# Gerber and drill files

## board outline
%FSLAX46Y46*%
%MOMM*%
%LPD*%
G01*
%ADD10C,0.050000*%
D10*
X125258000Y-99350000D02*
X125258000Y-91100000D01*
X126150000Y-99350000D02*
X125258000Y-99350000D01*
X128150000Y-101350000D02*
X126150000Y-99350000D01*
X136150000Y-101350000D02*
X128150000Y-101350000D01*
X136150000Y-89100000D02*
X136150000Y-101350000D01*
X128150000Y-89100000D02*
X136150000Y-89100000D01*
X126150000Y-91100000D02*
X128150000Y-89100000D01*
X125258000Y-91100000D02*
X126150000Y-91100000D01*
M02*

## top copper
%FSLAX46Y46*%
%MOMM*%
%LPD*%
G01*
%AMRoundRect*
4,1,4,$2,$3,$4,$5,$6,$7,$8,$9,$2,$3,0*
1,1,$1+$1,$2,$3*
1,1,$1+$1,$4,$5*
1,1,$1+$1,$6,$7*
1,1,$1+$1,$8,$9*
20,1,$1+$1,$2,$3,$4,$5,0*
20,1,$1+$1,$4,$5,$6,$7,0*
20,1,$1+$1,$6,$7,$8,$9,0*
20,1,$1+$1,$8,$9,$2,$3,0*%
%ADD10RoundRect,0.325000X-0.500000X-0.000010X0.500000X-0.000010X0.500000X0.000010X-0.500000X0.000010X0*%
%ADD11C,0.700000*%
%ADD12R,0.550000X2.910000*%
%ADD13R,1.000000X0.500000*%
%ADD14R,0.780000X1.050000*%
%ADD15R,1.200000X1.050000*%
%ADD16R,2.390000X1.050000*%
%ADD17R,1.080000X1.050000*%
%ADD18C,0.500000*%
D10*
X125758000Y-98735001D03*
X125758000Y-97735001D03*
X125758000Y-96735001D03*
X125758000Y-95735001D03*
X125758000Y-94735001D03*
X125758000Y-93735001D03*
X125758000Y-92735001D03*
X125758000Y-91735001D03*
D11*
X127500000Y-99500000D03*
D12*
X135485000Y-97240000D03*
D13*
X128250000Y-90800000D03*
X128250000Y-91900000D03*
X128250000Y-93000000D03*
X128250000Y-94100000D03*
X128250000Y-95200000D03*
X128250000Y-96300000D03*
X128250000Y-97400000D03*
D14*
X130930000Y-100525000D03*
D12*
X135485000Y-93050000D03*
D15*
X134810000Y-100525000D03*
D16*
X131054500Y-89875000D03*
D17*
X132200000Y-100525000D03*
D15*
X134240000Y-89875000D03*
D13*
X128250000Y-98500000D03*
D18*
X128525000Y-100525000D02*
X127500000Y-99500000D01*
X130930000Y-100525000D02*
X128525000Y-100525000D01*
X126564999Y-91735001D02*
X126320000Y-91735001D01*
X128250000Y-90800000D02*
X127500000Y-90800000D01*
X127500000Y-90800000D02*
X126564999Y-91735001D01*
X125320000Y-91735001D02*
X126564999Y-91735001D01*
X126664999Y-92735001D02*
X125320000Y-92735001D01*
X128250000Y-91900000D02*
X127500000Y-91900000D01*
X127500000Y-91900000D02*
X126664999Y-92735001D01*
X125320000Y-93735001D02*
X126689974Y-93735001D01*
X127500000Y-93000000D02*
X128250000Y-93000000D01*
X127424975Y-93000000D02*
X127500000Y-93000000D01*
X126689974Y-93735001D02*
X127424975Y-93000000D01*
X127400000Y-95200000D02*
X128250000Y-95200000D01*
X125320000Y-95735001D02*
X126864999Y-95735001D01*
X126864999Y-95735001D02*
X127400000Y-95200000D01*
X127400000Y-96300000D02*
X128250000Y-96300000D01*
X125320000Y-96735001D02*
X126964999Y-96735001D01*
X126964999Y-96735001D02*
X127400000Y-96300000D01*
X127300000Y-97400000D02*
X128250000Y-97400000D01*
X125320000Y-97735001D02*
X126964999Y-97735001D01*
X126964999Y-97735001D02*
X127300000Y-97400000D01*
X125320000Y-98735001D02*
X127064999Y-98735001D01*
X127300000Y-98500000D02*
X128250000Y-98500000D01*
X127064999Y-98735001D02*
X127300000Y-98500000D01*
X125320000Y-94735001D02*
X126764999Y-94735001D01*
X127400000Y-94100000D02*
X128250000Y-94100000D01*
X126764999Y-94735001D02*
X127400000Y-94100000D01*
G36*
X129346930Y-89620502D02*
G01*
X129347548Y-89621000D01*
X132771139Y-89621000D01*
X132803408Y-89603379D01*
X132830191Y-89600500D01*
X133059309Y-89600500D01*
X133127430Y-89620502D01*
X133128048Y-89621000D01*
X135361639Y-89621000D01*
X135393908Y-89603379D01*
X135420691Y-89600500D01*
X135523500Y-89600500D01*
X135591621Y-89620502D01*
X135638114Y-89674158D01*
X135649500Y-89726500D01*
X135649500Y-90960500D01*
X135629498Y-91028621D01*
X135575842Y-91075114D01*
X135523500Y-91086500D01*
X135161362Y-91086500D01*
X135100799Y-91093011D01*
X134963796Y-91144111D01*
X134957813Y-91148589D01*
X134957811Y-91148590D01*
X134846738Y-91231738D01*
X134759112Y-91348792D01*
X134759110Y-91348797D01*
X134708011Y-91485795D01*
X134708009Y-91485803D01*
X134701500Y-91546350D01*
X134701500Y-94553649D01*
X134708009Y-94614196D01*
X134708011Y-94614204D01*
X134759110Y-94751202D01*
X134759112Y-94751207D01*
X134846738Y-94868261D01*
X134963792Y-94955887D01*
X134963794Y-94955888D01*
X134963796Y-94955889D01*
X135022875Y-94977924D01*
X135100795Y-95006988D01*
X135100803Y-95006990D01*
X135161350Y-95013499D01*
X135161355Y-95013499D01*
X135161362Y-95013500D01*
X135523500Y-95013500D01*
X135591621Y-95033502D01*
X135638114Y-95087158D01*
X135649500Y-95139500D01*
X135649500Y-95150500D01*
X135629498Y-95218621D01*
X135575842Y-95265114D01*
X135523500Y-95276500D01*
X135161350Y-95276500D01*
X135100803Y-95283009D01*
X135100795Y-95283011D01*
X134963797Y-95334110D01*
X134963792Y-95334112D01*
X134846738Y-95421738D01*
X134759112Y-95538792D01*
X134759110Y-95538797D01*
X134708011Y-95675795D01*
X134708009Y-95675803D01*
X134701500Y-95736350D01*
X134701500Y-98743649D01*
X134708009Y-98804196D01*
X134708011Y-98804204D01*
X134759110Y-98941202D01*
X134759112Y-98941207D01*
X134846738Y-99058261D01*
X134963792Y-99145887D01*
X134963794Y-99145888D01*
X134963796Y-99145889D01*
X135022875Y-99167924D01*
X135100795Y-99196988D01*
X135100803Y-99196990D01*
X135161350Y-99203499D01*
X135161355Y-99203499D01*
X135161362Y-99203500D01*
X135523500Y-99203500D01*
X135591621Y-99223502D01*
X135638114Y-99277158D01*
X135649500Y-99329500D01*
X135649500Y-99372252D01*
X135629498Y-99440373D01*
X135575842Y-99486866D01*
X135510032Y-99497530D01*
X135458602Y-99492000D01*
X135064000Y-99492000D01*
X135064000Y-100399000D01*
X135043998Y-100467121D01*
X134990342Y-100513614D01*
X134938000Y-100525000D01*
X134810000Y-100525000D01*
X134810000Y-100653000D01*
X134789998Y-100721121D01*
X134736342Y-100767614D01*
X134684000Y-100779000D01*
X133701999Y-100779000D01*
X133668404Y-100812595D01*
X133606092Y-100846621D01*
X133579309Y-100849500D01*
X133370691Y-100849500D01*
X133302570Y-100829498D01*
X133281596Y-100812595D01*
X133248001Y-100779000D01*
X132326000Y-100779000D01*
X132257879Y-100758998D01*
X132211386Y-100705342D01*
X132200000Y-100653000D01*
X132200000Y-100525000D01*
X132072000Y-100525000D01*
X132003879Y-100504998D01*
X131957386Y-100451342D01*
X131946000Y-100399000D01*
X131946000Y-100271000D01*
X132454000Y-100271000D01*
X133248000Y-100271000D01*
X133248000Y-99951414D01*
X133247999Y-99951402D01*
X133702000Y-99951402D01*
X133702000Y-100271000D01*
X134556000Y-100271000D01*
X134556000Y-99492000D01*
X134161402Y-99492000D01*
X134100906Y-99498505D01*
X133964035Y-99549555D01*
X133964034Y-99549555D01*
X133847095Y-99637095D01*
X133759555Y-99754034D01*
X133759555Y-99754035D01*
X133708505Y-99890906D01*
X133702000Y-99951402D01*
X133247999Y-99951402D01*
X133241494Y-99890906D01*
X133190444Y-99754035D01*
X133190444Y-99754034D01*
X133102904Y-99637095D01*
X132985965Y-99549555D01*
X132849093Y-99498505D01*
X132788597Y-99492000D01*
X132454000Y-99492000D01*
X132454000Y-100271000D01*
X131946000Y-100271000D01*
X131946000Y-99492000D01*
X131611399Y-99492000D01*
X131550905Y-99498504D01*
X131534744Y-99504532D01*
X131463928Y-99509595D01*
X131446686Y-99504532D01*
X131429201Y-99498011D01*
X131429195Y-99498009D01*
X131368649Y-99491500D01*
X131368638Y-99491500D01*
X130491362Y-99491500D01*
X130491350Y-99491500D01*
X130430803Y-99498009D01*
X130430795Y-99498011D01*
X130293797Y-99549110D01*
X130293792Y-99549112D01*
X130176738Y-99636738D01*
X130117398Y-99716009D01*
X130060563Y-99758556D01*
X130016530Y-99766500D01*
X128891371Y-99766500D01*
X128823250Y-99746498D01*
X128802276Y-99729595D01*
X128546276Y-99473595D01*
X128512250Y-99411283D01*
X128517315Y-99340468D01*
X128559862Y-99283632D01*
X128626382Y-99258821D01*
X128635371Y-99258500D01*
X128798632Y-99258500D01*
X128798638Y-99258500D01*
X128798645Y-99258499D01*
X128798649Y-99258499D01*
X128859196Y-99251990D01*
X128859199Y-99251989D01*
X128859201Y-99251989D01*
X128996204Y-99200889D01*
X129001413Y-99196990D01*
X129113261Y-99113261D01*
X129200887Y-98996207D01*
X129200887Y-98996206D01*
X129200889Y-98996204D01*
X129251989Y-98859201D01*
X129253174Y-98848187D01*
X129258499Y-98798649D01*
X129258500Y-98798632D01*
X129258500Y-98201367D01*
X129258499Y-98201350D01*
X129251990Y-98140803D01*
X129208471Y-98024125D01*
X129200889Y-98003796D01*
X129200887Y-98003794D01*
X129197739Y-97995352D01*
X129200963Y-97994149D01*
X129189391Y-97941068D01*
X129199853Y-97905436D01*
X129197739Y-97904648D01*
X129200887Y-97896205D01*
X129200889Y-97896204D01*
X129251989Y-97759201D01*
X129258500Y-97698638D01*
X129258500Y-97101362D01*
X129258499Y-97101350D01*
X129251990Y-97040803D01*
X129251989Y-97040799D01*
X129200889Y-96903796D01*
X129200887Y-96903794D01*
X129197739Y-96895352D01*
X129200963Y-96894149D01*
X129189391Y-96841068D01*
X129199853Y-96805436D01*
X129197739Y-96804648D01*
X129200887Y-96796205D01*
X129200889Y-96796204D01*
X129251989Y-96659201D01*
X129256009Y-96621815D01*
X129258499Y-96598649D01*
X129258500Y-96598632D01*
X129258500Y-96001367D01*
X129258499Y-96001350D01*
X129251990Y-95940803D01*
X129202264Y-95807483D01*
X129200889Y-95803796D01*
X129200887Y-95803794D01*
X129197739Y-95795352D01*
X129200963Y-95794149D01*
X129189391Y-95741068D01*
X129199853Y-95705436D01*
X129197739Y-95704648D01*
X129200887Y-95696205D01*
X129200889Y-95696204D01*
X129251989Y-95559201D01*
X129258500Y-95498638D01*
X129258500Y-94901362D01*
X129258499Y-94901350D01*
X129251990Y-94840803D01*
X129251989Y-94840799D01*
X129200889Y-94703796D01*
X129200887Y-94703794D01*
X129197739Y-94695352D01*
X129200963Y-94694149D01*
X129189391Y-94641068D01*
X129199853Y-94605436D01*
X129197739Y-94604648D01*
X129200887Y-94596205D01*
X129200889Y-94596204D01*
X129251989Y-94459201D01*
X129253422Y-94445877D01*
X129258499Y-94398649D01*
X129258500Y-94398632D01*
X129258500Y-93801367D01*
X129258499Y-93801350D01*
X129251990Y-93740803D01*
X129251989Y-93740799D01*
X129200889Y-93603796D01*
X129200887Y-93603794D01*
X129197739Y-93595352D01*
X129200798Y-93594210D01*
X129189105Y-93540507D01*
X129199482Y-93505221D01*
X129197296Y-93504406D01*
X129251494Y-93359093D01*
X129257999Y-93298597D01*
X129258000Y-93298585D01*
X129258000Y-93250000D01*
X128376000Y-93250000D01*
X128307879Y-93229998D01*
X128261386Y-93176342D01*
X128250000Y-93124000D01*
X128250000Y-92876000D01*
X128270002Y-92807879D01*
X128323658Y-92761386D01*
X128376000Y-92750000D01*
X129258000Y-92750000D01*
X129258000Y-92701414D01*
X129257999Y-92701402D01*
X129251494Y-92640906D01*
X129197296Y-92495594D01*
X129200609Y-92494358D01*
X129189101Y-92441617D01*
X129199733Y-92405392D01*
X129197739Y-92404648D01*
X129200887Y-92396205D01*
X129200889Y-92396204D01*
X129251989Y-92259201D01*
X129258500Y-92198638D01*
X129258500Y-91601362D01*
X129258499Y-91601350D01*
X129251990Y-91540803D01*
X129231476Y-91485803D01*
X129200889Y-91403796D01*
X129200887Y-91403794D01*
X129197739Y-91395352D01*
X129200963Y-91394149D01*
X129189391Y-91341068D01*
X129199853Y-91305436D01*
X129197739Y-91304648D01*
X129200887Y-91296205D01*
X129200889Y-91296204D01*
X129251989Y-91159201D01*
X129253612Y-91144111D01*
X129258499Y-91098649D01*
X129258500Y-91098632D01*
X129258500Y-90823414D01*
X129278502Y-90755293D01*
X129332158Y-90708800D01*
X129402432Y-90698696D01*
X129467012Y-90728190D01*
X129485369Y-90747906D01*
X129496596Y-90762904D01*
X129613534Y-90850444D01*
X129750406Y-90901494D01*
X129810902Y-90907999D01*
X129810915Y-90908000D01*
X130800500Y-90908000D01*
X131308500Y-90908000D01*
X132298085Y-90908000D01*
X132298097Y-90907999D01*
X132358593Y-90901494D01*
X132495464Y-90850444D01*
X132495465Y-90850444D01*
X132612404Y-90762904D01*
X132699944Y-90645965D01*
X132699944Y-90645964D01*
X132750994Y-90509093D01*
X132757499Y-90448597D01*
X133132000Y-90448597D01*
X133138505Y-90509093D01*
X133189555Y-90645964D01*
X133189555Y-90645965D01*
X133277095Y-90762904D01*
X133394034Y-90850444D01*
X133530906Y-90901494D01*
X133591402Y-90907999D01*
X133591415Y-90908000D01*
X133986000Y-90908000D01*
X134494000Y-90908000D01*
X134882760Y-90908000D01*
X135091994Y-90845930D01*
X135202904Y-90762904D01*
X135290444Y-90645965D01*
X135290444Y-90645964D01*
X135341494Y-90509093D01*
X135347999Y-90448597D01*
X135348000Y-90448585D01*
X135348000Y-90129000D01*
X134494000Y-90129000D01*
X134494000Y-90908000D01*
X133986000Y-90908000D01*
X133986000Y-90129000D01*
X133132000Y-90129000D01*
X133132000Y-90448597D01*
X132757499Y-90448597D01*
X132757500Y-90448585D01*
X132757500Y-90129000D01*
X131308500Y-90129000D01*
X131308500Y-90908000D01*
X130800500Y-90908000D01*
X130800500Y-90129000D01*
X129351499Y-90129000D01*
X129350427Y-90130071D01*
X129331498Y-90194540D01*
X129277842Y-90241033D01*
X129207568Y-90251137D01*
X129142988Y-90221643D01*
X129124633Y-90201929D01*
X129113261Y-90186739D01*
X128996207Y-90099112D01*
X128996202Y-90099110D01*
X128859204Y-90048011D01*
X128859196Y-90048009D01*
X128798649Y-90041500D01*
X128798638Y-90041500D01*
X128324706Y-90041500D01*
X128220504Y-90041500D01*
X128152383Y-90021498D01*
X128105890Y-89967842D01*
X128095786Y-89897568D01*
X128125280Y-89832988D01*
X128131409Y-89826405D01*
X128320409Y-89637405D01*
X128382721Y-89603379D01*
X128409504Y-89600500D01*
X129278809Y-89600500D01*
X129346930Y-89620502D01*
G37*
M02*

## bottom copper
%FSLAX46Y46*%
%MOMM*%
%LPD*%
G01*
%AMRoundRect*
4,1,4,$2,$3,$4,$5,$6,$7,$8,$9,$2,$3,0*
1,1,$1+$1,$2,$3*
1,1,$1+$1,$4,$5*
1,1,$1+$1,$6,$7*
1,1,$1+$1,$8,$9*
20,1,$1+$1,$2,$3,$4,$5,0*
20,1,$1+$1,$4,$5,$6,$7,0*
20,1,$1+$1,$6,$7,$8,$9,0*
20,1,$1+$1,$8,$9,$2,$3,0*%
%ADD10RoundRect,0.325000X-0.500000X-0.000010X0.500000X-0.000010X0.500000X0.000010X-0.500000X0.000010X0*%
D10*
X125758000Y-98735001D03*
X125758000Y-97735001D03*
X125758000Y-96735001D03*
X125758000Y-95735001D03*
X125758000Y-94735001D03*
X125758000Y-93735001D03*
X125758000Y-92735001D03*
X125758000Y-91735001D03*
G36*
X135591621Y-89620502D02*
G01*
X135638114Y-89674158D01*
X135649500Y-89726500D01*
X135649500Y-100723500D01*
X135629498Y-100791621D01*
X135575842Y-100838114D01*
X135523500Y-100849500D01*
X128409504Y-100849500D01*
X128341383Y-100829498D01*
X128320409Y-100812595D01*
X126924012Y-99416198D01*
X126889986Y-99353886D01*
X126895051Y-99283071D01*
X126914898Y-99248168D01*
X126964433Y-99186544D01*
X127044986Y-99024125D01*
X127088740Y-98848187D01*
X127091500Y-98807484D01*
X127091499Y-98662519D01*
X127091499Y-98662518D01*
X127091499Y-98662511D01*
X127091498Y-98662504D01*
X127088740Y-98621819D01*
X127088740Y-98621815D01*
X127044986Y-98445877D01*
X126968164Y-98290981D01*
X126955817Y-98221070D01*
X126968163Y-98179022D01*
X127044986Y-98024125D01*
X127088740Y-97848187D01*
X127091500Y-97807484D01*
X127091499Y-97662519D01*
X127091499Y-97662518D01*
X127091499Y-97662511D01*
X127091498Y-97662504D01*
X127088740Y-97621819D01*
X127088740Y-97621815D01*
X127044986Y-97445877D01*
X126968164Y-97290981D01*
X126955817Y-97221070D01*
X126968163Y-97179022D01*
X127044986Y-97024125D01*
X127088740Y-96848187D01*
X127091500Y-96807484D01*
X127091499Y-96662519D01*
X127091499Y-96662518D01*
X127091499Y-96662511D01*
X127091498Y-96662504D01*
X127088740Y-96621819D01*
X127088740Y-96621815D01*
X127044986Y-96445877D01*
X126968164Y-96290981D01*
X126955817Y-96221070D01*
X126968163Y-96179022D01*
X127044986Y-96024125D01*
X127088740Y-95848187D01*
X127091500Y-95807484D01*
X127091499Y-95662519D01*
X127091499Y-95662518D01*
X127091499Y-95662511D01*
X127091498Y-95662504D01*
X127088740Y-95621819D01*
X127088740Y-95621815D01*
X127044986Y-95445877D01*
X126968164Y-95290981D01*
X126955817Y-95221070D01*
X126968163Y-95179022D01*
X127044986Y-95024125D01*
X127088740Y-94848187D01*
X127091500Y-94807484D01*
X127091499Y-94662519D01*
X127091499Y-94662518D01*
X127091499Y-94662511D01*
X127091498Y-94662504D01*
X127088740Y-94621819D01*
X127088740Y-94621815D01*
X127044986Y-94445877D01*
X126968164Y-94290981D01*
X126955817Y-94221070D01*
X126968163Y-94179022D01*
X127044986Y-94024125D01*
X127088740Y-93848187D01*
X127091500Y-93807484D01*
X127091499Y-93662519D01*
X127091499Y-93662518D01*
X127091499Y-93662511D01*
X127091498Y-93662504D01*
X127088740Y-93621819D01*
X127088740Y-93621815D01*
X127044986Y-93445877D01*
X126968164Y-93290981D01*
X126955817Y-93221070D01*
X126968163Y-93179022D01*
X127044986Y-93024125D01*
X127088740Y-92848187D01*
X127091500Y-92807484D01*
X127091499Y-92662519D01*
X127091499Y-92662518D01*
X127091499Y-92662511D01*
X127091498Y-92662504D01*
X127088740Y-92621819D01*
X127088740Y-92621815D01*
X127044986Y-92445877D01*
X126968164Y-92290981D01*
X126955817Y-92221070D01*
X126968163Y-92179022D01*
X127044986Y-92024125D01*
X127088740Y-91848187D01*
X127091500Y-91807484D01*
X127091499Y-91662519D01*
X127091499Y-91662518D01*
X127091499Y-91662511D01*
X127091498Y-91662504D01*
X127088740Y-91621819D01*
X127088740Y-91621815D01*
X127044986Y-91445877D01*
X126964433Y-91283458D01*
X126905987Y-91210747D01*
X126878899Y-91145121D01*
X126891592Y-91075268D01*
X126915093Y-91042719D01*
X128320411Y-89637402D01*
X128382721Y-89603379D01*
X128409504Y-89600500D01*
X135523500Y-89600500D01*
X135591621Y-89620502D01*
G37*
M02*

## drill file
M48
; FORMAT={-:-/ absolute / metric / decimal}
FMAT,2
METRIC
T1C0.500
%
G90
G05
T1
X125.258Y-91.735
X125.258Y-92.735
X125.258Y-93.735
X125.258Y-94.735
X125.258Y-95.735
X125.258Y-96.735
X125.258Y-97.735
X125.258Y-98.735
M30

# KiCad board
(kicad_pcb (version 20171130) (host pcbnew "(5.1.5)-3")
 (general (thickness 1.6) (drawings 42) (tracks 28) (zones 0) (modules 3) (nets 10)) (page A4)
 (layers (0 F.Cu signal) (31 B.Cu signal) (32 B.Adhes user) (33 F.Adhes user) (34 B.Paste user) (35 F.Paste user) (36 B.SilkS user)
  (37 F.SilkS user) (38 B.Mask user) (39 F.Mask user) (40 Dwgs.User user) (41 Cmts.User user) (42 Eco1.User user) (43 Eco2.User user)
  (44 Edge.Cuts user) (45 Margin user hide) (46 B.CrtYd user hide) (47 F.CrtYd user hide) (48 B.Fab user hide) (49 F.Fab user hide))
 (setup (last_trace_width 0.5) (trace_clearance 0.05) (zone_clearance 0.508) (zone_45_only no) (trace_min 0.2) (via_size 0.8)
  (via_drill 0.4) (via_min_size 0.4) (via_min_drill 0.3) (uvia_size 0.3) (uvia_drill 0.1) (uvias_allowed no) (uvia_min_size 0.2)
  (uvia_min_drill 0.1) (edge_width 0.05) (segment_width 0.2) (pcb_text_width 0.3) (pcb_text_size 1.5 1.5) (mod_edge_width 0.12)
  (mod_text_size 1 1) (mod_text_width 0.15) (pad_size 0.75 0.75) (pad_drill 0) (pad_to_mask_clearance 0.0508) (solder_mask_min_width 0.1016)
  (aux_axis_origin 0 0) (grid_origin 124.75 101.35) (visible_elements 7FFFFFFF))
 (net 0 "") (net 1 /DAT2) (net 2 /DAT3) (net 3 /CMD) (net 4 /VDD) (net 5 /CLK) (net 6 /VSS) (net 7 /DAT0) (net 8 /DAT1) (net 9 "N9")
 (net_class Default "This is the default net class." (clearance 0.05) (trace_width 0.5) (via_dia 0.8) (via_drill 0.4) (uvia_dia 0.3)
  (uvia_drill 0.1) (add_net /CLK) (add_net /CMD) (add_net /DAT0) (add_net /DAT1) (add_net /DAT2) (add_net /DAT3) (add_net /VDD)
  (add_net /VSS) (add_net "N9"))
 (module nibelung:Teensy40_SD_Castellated (layer F.Cu) (at 125.258 91.735001)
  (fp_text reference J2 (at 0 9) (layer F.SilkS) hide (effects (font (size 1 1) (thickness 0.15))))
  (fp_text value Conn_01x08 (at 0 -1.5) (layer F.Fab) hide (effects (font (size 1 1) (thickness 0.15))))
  (pad 8 thru_hole roundrect (at 0 7) (size 1.65 0.65) (drill 0.5 (offset 0.5 0)) (layers *.Cu *.Mask) (roundrect_rratio 0.5) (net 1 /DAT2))
  (pad 7 thru_hole roundrect (at 0 6) (size 1.65 0.65) (drill 0.5 (offset 0.5 0)) (layers *.Cu *.Mask) (roundrect_rratio 0.5) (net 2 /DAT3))
  (pad 6 thru_hole roundrect (at 0 5) (size 1.65 0.65) (drill 0.5 (offset 0.5 0)) (layers *.Cu *.Mask) (roundrect_rratio 0.5) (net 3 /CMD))
  (pad 5 thru_hole roundrect (at 0 4) (size 1.65 0.65) (drill 0.5 (offset 0.5 0)) (layers *.Cu *.Mask) (roundrect_rratio 0.5) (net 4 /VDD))
  (pad 4 thru_hole roundrect (at 0 3) (size 1.65 0.65) (drill 0.5 (offset 0.5 0)) (layers *.Cu *.Mask) (roundrect_rratio 0.5) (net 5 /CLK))
  (pad 3 thru_hole roundrect (at 0 2) (size 1.65 0.65) (drill 0.5 (offset 0.5 0)) (layers *.Cu *.Mask) (roundrect_rratio 0.5) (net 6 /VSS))
  (pad 2 thru_hole roundrect (at 0 1) (size 1.65 0.65) (drill 0.5 (offset 0.5 0)) (layers *.Cu *.Mask) (roundrect_rratio 0.5) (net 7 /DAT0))
  (pad 1 thru_hole roundrect (at 0 0) (size 1.65 0.65) (drill 0.5 (offset 0.5 0)) (layers *.Cu *.Mask) (roundrect_rratio 0.5) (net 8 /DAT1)))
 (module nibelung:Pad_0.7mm (layer F.Cu) (at 127.5 99.5)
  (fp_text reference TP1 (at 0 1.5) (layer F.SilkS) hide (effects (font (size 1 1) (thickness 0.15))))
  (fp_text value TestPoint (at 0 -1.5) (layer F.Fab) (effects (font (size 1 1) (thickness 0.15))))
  (pad 1 smd circle (at 0 0) (size 0.7 0.7) (layers F.Cu F.Paste F.Mask) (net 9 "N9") (solder_mask_margin 0.03)))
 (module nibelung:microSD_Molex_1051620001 (layer F.Cu) (at 127.75 98.75 270)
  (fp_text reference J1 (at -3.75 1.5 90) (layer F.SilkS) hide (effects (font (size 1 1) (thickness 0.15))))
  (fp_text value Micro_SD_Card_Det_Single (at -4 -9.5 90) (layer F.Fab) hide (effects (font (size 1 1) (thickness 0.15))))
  (pad 11 smd rect (at -2.96 -7.46 270) (size 2.91 0.55) (drill (offset 1.45 -0.275)) (layers F.Cu F.Paste F.Mask))
  (pad 8 smd rect (at -7.95 -0.5 270) (size 0.5 1) (layers F.Cu F.Paste F.Mask) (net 8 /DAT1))
  (pad 7 smd rect (at -6.85 -0.5 270) (size 0.5 1) (layers F.Cu F.Paste F.Mask) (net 7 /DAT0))
  (pad 6 smd rect (at -5.75 -0.5 270) (size 0.5 1) (layers F.Cu F.Paste F.Mask) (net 6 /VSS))
  (pad 5 smd rect (at -4.65 -0.5 270) (size 0.5 1) (layers F.Cu F.Paste F.Mask) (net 5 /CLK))
  (pad 4 smd rect (at -3.55 -0.5 270) (size 0.5 1) (layers F.Cu F.Paste F.Mask) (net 4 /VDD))
  (pad 3 smd rect (at -2.45 -0.5 270) (size 0.5 1) (layers F.Cu F.Paste F.Mask) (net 3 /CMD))
  (pad 2 smd rect (at -1.35 -0.5 270) (size 0.5 1) (layers F.Cu F.Paste F.Mask) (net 2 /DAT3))
  (pad 9 smd rect (at 1.775 -3.18 270) (size 1.05 0.78) (layers F.Cu F.Paste F.Mask) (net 9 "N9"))
  (pad 11 smd rect (at -7.15 -7.46 270) (size 2.91 0.55) (drill (offset 1.45 -0.275)) (layers F.Cu F.Paste F.Mask))
  (pad 10 smd rect (at 1.25 -6.46 270) (size 1.05 1.2) (drill (offset 0.525 -0.6)) (layers F.Cu F.Paste F.Mask) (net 6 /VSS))
  (pad 10 smd rect (at -9.4 -2.11 270) (size 1.05 2.39) (drill (offset 0.525 -1.1945)) (layers F.Cu F.Paste F.Mask) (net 6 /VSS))
  (pad 10 smd rect (at 1.25 -3.91 270) (size 1.05 1.08) (drill (offset 0.525 -0.54)) (layers F.Cu F.Paste F.Mask) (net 6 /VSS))
  (pad 10 smd rect (at -9.4 -5.89 270) (size 1.05 1.2) (drill (offset 0.525 -0.6)) (layers F.Cu F.Paste F.Mask) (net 6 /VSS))
  (pad 1 smd rect (at -0.25 -0.5 270) (size 0.5 1) (layers F.Cu F.Paste F.Mask) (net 1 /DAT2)))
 (gr_line (start 125.258 99.35) (end 125.258 91.1) (layer Edge.Cuts) (width 0.05))
 (gr_line (start 126.15 99.35) (end 125.258 99.35) (layer Edge.Cuts) (width 0.05))
 (gr_line (start 128.15 101.35) (end 126.15 99.35) (layer Edge.Cuts) (width 0.05))
 (gr_line (start 136.15 101.35) (end 128.15 101.35) (layer Edge.Cuts) (width 0.05))
 (gr_line (start 136.15 89.1) (end 136.15 101.35) (layer Edge.Cuts) (width 0.05))
 (gr_line (start 128.15 89.1) (end 136.15 89.1) (layer Edge.Cuts) (width 0.05))
 (gr_line (start 126.15 91.1) (end 128.15 89.1) (layer Edge.Cuts) (width 0.05))
 (gr_line (start 125.258 91.1) (end 126.15 91.1) (layer Edge.Cuts) (width 0.05))
 (segment (start 128.525 100.525) (end 127.5 99.5) (width 0.5) (layer F.Cu) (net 9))
 (segment (start 130.93 100.525) (end 128.525 100.525) (width 0.5) (layer F.Cu) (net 9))
 (segment (start 126.564999 91.735001) (end 126.32 91.735001) (width 0.5) (layer F.Cu) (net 8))
 (segment (start 128.25 90.8) (end 127.5 90.8) (width 0.5) (layer F.Cu) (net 8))
 (segment (start 127.5 90.8) (end 126.564999 91.735001) (width 0.5) (layer F.Cu) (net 8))
 (segment (start 125.32 91.735001) (end 126.564999 91.735001) (width 0.5) (layer F.Cu) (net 8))
 (segment (start 126.664999 92.735001) (end 125.32 92.735001) (width 0.5) (layer F.Cu) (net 7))
 (segment (start 128.25 91.9) (end 127.5 91.9) (width 0.5) (layer F.Cu) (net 7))
 (segment (start 127.5 91.9) (end 126.664999 92.735001) (width 0.5) (layer F.Cu) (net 7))
 (segment (start 125.32 93.735001) (end 126.689974 93.735001) (width 0.5) (layer F.Cu) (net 6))
 (segment (start 127.5 93) (end 128.25 93) (width 0.5) (layer F.Cu) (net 6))
 (segment (start 127.424975 93) (end 127.5 93) (width 0.5) (layer F.Cu) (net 6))
 (segment (start 126.689974 93.735001) (end 127.424975 93) (width 0.5) (layer F.Cu) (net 6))
 (segment (start 127.4 95.2) (end 128.25 95.2) (width 0.5) (layer F.Cu) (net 4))
 (segment (start 125.32 95.735001) (end 126.864999 95.735001) (width 0.5) (layer F.Cu) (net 4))
 (segment (start 126.864999 95.735001) (end 127.4 95.2) (width 0.5) (layer F.Cu) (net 4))
 (segment (start 127.4 96.3) (end 128.25 96.3) (width 0.5) (layer F.Cu) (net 3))
 (segment (start 125.32 96.735001) (end 126.964999 96.735001) (width 0.5) (layer F.Cu) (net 3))
 (segment (start 126.964999 96.735001) (end 127.4 96.3) (width 0.5) (layer F.Cu) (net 3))
 (segment (start 127.3 97.4) (end 128.25 97.4) (width 0.5) (layer F.Cu) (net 2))
 (segment (start 125.32 97.735001) (end 126.964999 97.735001) (width 0.5) (layer F.Cu) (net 2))
 (segment (start 126.964999 97.735001) (end 127.3 97.4) (width 0.5) (layer F.Cu) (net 2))
 (segment (start 125.32 98.735001) (end 127.064999 98.735001) (width 0.5) (layer F.Cu) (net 1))
 (segment (start 127.3 98.5) (end 128.25 98.5) (width 0.5) (layer F.Cu) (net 1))
 (segment (start 127.064999 98.735001) (end 127.3 98.5) (width 0.5) (layer F.Cu) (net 1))
 (segment (start 125.32 94.735001) (end 126.764999 94.735001) (width 0.5) (layer F.Cu) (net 5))
 (segment (start 127.4 94.1) (end 128.25 94.1) (width 0.5) (layer F.Cu) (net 5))
 (segment (start 126.764999 94.735001) (end 127.4 94.1) (width 0.5) (layer F.Cu) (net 5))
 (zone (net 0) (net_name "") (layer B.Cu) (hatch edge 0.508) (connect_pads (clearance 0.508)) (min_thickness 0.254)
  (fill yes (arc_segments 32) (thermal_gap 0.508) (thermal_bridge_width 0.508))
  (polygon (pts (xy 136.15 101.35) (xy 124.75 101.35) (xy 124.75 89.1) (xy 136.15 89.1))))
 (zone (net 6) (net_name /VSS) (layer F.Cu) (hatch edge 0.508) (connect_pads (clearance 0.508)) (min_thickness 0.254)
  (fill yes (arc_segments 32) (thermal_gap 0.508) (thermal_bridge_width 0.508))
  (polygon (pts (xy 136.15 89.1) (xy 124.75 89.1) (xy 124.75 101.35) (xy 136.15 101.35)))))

